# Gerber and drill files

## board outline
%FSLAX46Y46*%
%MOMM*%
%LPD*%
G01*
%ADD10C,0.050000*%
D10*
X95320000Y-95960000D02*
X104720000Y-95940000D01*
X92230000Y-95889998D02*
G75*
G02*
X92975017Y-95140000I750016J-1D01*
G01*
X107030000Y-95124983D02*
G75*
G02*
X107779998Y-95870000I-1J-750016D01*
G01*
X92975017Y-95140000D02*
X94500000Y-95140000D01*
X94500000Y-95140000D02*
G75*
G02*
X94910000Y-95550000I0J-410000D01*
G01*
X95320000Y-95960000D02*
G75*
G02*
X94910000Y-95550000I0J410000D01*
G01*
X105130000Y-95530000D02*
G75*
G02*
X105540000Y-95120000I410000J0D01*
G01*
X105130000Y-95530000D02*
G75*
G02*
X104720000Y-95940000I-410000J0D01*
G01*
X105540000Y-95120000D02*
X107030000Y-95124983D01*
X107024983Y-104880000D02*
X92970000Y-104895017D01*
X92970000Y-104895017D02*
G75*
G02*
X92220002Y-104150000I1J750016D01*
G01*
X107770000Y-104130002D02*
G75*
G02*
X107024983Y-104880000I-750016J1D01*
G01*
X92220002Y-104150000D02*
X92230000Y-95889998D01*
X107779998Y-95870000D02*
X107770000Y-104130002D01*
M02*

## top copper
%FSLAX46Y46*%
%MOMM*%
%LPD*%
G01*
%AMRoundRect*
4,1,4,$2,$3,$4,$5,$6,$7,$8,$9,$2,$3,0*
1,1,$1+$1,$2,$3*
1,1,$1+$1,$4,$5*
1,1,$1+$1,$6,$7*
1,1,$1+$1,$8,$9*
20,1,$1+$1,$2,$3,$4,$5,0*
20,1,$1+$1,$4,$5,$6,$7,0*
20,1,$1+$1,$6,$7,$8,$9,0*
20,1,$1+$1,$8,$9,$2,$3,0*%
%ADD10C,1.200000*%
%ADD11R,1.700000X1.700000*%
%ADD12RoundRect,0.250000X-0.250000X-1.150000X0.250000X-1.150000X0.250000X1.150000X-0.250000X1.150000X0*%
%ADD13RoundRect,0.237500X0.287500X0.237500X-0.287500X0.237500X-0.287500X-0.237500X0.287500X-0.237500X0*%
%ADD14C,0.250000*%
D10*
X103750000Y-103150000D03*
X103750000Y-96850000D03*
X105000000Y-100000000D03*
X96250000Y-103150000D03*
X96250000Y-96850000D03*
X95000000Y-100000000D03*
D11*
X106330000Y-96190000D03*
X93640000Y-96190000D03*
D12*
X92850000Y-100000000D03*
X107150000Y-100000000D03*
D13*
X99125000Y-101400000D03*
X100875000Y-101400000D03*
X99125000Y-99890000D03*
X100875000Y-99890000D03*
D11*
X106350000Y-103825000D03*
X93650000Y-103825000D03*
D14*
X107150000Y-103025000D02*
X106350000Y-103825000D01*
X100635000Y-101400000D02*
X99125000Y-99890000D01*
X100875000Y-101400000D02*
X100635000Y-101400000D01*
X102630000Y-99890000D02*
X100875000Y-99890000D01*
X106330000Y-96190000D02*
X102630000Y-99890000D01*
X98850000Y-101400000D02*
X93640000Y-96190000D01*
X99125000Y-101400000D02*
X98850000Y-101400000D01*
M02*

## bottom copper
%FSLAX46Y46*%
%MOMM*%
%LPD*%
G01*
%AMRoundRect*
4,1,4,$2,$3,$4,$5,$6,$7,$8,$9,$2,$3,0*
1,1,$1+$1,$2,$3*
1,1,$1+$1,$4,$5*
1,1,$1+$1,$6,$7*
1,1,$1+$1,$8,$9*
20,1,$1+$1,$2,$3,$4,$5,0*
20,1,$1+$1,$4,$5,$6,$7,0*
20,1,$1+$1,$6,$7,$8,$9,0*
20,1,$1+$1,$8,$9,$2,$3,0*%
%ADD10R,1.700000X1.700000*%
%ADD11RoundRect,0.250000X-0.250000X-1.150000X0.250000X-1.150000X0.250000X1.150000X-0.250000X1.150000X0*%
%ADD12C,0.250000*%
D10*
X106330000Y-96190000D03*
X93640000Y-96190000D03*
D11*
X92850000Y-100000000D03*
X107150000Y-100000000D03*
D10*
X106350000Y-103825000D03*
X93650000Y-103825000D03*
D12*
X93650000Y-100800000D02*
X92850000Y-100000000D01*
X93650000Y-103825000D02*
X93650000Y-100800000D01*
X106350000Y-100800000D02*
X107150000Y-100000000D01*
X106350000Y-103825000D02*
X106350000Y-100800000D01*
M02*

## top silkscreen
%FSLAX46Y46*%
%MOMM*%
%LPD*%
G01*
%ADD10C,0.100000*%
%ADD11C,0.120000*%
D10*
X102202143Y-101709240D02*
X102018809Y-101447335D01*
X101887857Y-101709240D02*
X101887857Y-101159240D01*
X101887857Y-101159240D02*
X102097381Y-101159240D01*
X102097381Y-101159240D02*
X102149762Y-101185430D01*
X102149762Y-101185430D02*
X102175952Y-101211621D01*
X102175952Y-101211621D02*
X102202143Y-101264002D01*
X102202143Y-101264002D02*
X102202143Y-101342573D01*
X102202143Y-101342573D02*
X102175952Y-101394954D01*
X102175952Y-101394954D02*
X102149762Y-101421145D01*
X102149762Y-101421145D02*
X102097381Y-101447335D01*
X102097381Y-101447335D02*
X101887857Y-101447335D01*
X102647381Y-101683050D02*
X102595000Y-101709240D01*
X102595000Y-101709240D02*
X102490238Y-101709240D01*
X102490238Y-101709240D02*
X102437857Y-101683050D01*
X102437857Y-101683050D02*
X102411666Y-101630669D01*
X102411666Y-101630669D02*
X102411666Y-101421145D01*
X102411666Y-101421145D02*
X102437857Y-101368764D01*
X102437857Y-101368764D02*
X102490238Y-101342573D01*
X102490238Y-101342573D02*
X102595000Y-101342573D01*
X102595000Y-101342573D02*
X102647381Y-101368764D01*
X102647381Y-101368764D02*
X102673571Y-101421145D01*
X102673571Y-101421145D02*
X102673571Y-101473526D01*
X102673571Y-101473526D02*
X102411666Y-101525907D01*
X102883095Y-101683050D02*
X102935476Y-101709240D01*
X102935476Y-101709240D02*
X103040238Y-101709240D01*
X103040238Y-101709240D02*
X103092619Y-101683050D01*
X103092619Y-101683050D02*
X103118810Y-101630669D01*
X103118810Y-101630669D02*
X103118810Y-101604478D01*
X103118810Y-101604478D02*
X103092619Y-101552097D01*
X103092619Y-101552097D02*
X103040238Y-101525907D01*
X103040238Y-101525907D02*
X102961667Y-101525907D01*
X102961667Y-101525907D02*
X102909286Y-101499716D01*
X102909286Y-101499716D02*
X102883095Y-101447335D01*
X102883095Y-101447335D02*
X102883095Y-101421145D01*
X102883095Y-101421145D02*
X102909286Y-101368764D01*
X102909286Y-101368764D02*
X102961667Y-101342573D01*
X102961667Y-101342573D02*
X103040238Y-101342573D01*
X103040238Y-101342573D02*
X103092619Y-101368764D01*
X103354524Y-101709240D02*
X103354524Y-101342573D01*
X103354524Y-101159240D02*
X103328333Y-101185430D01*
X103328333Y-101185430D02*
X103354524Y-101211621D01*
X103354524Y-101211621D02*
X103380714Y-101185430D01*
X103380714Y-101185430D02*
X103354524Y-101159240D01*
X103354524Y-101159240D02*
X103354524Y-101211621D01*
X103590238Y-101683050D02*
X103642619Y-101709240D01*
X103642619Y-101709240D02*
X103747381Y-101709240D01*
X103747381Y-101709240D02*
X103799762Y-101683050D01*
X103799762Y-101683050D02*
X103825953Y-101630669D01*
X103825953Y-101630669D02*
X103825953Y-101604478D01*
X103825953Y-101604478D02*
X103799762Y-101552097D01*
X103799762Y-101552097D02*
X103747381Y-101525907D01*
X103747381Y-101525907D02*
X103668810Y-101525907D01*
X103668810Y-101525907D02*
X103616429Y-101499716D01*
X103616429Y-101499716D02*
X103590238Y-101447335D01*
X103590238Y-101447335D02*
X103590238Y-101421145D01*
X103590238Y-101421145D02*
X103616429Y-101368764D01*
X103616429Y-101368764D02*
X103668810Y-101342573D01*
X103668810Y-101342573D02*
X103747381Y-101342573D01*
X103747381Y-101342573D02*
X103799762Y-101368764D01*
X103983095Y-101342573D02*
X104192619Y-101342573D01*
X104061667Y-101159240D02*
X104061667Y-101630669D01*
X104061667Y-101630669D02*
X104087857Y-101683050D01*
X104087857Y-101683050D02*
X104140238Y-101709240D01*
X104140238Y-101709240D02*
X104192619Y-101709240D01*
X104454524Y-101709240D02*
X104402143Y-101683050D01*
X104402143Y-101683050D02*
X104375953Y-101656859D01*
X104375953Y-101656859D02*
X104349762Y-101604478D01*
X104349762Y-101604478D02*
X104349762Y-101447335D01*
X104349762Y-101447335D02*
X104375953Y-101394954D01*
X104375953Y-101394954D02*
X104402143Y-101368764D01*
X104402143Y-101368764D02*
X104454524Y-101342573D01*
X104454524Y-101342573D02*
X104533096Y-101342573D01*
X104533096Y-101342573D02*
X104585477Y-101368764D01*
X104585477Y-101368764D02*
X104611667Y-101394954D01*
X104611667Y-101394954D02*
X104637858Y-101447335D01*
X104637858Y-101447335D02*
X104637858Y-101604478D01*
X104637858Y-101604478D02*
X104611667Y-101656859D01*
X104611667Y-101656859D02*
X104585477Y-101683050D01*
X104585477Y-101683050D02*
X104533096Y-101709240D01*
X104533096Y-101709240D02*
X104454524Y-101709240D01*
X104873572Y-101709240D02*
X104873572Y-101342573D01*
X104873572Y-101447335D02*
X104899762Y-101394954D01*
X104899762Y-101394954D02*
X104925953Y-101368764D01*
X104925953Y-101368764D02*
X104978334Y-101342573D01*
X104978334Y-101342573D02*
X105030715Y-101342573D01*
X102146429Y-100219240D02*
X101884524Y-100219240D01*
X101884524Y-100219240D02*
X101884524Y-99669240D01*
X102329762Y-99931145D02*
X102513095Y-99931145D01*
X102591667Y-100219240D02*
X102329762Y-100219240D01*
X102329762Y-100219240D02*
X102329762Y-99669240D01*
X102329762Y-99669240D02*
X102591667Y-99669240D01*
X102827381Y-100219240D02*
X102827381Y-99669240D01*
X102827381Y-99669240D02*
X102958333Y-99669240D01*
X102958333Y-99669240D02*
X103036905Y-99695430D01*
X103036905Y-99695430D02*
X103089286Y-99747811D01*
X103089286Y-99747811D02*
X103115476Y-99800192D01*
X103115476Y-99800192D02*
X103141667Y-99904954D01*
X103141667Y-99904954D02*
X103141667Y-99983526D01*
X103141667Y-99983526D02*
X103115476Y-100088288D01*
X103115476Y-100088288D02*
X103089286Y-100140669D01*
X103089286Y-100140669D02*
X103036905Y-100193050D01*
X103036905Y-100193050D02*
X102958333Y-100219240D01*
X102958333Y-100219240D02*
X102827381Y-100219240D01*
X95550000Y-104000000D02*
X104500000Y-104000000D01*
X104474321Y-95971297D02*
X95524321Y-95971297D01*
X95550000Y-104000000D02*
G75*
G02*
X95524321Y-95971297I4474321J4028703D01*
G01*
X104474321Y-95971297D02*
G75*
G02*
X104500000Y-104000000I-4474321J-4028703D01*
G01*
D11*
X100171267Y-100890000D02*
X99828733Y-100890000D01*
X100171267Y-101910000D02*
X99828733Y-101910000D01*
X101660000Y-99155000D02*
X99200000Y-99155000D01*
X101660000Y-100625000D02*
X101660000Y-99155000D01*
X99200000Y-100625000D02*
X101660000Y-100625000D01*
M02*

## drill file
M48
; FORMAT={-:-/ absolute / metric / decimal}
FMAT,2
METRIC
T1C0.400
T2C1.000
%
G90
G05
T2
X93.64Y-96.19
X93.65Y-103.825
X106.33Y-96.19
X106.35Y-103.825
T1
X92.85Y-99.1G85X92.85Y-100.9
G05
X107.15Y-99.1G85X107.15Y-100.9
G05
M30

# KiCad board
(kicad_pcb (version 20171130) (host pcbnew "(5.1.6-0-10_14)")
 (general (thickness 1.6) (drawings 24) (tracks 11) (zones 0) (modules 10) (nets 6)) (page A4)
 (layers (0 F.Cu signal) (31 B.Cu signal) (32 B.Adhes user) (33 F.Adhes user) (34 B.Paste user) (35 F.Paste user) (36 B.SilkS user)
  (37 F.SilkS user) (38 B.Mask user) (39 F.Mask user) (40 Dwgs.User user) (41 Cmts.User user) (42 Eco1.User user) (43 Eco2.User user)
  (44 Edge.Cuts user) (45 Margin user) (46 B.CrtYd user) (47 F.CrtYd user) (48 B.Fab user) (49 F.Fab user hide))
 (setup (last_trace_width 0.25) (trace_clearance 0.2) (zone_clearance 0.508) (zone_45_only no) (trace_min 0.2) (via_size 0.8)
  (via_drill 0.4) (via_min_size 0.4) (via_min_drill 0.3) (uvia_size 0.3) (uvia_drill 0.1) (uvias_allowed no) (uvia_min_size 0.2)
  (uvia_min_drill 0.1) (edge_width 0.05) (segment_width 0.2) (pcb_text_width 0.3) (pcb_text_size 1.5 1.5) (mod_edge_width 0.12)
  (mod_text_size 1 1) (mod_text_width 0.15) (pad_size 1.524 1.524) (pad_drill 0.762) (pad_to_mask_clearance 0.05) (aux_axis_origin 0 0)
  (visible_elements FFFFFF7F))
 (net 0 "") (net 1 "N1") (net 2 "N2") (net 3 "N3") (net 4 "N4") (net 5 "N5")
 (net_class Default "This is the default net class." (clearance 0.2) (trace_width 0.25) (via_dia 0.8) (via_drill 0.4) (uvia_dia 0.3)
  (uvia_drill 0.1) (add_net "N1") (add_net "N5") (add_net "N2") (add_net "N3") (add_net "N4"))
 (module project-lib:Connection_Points (layer F.Cu) (at 100 100)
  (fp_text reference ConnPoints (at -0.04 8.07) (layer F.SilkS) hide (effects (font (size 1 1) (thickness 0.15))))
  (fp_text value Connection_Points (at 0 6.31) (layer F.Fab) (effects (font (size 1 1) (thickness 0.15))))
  (pad "" smd circle (at 3.75 3.15) (size 1.2 1.2) (layers F.Cu F.Paste F.Mask))
  (pad "" smd circle (at 3.75 -3.15) (size 1.2 1.2) (layers F.Cu F.Paste F.Mask))
  (pad "" smd circle (at 5 0) (size 1.2 1.2) (layers F.Cu F.Paste F.Mask))
  (pad "" smd circle (at -3.75 3.15) (size 1.2 1.2) (layers F.Cu F.Paste F.Mask))
  (pad "" smd circle (at -3.75 -3.15) (size 1.2 1.2) (layers F.Cu F.Paste F.Mask))
  (pad "" smd circle (at -5 0) (size 1.2 1.2) (layers F.Cu F.Paste F.Mask)))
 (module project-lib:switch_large (layer B.Cu) (at 100 103.1 180)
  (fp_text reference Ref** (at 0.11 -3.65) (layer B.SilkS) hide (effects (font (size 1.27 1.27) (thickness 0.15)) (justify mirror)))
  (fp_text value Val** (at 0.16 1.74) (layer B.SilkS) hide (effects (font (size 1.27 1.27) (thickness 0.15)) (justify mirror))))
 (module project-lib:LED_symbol (layer B.Cu) (at 100.02 96.94)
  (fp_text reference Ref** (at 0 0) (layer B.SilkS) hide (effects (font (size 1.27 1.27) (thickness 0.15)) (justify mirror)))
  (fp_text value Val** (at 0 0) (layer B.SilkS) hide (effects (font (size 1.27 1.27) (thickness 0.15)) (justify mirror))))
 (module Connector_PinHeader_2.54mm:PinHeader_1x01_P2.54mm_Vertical (layer F.Cu) (at 106.33 96.19)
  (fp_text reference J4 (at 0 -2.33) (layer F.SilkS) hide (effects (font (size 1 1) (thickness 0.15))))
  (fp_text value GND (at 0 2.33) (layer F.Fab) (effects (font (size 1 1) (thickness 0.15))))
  (pad 1 thru_hole rect (at 0 0) (size 1.7 1.7) (drill 1) (layers *.Cu *.Mask) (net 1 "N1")))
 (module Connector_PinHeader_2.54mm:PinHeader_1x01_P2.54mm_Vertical (layer F.Cu) (at 93.64 96.19)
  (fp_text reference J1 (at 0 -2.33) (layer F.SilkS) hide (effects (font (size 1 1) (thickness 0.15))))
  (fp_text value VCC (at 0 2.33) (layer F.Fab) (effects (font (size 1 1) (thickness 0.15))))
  (pad 1 thru_hole rect (at 0 0) (size 1.7 1.7) (drill 1) (layers *.Cu *.Mask) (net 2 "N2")))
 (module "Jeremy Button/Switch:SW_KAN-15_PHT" (layer F.Cu) (at 100 100)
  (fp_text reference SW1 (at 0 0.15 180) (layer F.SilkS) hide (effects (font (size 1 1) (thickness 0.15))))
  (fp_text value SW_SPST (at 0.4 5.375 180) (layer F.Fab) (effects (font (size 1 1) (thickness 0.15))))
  (fp_line (start -4.45 4) (end 4.5 4) (layer F.SilkS) (width 0.1))
  (fp_line (start 4.474321 -4.028703) (end -4.475679 -4.028703) (layer F.SilkS) (width 0.1))
  (fp_arc (start 0.024321 -0.028703) (end -4.475679 -4.028703) (angle -83.63358372) (layer F.SilkS) (width 0.1))
  (fp_arc (start 0 0) (end 4.5 4) (angle -83.63358372) (layer F.SilkS) (width 0.1))
  (pad 1 thru_hole roundrect (at -7.15 0) (size 1 2.8) (drill oval 0.4 2.2) (layers *.Cu *.Mask) (roundrect_rratio 0.25) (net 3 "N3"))
  (pad 2 thru_hole roundrect (at 7.15 0) (size 1 2.8) (drill oval 0.4 2.2) (layers *.Cu *.Mask) (roundrect_rratio 0.25) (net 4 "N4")))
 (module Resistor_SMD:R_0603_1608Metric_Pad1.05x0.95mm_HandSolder (layer F.Cu) (at 100 101.4 180)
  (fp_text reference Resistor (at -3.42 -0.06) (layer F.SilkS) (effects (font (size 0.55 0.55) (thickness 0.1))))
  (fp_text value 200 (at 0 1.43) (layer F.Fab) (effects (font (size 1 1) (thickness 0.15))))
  (fp_line (start -0.171267 0.51) (end 0.171267 0.51) (layer F.SilkS) (width 0.12))
  (fp_line (start -0.171267 -0.51) (end 0.171267 -0.51) (layer F.SilkS) (width 0.12))
  (pad 2 smd roundrect (at 0.875 0 180) (size 1.05 0.95) (layers F.Cu F.Paste F.Mask) (roundrect_rratio 0.25) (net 2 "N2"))
  (pad 1 smd roundrect (at -0.875 0 180) (size 1.05 0.95) (layers F.Cu F.Paste F.Mask) (roundrect_rratio 0.25) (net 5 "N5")))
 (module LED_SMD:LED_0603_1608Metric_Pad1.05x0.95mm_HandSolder (layer F.Cu) (at 100 99.89 180)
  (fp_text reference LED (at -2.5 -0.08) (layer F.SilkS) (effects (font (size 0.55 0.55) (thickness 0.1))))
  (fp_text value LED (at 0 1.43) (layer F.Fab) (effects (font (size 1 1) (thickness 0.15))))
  (fp_line (start -1.66 0.735) (end 0.8 0.735) (layer F.SilkS) (width 0.12))
  (fp_line (start -1.66 -0.735) (end -1.66 0.735) (layer F.SilkS) (width 0.12))
  (fp_line (start 0.8 -0.735) (end -1.66 -0.735) (layer F.SilkS) (width 0.12))
  (pad 2 smd roundrect (at 0.875 0 180) (size 1.05 0.95) (layers F.Cu F.Paste F.Mask) (roundrect_rratio 0.25) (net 5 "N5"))
  (pad 1 smd roundrect (at -0.875 0 180) (size 1.05 0.95) (layers F.Cu F.Paste F.Mask) (roundrect_rratio 0.25) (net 1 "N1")))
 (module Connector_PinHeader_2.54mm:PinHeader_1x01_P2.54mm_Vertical (layer F.Cu) (at 106.35 103.825 180)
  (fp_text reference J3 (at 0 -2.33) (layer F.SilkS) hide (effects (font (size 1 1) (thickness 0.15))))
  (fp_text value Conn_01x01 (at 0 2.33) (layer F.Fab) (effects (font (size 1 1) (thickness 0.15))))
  (pad 1 thru_hole rect (at 0 0 180) (size 1.7 1.7) (drill 1) (layers *.Cu *.Mask) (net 4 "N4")))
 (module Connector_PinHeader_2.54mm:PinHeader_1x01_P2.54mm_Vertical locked (layer F.Cu) (at 93.65 103.825 90)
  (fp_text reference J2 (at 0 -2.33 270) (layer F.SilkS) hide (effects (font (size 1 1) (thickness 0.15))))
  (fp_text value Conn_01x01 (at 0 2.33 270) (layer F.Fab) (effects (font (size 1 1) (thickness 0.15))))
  (pad 1 thru_hole rect (at 0 0 90) (size 1.7 1.7) (drill 1) (layers *.Cu *.Mask) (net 3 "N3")))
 (gr_line (start 95.32 95.96) (end 104.72 95.94) (layer Edge.Cuts) (width 0.05))
 (gr_arc (start 92.980016 95.889999) (end 92.975017 95.14) (angle -89.6180338) (layer Edge.Cuts) (width 0.05))
 (gr_arc (start 107.029999 95.874999) (end 107.779998 95.87) (angle -89.6180338) (layer Edge.Cuts) (width 0.05))
 (gr_line (start 92.975017 95.14) (end 94.5 95.14) (layer Edge.Cuts) (width 0.05))
 (gr_arc (start 94.5 95.55) (end 94.91 95.55) (angle -90) (layer Edge.Cuts) (width 0.05))
 (gr_arc (start 95.32 95.55) (end 94.91 95.55) (angle -90) (layer Edge.Cuts) (width 0.05))
 (gr_arc (start 105.54 95.53) (end 105.54 95.12) (angle -90) (layer Edge.Cuts) (width 0.05))
 (gr_arc (start 104.72 95.53) (end 104.72 95.94) (angle -90) (layer Edge.Cuts) (width 0.05))
 (gr_line (start 105.54 95.12) (end 107.03 95.124983) (layer Edge.Cuts) (width 0.05))
 (gr_line (start 107.024983 104.88) (end 92.97 104.895017) (layer Edge.Cuts) (width 0.05))
 (gr_arc (start 92.970001 104.145001) (end 92.220002 104.15) (angle -89.6180338) (layer Edge.Cuts) (width 0.05))
 (gr_arc (start 107.019984 104.130001) (end 107.024983 104.88) (angle -89.61803328) (layer Edge.Cuts) (width 0.05))
 (gr_line (start 92.220002 104.15) (end 92.23 95.889998) (layer Edge.Cuts) (width 0.05))
 (gr_line (start 107.779998 95.87) (end 107.77 104.130002) (layer Edge.Cuts) (width 0.05))
 (segment (start 93.65 100.8) (end 92.85 100) (width 0.25) (layer B.Cu) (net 3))
 (segment (start 93.65 103.825) (end 93.65 100.8) (width 0.25) (layer B.Cu) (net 3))
 (segment (start 107.15 103.025) (end 106.35 103.825) (width 0.25) (layer F.Cu) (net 4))
 (segment (start 106.35 100.8) (end 107.15 100) (width 0.25) (layer B.Cu) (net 4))
 (segment (start 106.35 103.825) (end 106.35 100.8) (width 0.25) (layer B.Cu) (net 4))
 (segment (start 100.635 101.4) (end 99.125 99.89) (width 0.25) (layer F.Cu) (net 5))
 (segment (start 100.875 101.4) (end 100.635 101.4) (width 0.25) (layer F.Cu) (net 5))
 (segment (start 102.63 99.89) (end 100.875 99.89) (width 0.25) (layer F.Cu) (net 1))
 (segment (start 106.33 96.19) (end 102.63 99.89) (width 0.25) (layer F.Cu) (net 1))
 (segment (start 98.85 101.4) (end 93.64 96.19) (width 0.25) (layer F.Cu) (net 2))
 (segment (start 99.125 101.4) (end 98.85 101.4) (width 0.25) (layer F.Cu) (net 2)))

